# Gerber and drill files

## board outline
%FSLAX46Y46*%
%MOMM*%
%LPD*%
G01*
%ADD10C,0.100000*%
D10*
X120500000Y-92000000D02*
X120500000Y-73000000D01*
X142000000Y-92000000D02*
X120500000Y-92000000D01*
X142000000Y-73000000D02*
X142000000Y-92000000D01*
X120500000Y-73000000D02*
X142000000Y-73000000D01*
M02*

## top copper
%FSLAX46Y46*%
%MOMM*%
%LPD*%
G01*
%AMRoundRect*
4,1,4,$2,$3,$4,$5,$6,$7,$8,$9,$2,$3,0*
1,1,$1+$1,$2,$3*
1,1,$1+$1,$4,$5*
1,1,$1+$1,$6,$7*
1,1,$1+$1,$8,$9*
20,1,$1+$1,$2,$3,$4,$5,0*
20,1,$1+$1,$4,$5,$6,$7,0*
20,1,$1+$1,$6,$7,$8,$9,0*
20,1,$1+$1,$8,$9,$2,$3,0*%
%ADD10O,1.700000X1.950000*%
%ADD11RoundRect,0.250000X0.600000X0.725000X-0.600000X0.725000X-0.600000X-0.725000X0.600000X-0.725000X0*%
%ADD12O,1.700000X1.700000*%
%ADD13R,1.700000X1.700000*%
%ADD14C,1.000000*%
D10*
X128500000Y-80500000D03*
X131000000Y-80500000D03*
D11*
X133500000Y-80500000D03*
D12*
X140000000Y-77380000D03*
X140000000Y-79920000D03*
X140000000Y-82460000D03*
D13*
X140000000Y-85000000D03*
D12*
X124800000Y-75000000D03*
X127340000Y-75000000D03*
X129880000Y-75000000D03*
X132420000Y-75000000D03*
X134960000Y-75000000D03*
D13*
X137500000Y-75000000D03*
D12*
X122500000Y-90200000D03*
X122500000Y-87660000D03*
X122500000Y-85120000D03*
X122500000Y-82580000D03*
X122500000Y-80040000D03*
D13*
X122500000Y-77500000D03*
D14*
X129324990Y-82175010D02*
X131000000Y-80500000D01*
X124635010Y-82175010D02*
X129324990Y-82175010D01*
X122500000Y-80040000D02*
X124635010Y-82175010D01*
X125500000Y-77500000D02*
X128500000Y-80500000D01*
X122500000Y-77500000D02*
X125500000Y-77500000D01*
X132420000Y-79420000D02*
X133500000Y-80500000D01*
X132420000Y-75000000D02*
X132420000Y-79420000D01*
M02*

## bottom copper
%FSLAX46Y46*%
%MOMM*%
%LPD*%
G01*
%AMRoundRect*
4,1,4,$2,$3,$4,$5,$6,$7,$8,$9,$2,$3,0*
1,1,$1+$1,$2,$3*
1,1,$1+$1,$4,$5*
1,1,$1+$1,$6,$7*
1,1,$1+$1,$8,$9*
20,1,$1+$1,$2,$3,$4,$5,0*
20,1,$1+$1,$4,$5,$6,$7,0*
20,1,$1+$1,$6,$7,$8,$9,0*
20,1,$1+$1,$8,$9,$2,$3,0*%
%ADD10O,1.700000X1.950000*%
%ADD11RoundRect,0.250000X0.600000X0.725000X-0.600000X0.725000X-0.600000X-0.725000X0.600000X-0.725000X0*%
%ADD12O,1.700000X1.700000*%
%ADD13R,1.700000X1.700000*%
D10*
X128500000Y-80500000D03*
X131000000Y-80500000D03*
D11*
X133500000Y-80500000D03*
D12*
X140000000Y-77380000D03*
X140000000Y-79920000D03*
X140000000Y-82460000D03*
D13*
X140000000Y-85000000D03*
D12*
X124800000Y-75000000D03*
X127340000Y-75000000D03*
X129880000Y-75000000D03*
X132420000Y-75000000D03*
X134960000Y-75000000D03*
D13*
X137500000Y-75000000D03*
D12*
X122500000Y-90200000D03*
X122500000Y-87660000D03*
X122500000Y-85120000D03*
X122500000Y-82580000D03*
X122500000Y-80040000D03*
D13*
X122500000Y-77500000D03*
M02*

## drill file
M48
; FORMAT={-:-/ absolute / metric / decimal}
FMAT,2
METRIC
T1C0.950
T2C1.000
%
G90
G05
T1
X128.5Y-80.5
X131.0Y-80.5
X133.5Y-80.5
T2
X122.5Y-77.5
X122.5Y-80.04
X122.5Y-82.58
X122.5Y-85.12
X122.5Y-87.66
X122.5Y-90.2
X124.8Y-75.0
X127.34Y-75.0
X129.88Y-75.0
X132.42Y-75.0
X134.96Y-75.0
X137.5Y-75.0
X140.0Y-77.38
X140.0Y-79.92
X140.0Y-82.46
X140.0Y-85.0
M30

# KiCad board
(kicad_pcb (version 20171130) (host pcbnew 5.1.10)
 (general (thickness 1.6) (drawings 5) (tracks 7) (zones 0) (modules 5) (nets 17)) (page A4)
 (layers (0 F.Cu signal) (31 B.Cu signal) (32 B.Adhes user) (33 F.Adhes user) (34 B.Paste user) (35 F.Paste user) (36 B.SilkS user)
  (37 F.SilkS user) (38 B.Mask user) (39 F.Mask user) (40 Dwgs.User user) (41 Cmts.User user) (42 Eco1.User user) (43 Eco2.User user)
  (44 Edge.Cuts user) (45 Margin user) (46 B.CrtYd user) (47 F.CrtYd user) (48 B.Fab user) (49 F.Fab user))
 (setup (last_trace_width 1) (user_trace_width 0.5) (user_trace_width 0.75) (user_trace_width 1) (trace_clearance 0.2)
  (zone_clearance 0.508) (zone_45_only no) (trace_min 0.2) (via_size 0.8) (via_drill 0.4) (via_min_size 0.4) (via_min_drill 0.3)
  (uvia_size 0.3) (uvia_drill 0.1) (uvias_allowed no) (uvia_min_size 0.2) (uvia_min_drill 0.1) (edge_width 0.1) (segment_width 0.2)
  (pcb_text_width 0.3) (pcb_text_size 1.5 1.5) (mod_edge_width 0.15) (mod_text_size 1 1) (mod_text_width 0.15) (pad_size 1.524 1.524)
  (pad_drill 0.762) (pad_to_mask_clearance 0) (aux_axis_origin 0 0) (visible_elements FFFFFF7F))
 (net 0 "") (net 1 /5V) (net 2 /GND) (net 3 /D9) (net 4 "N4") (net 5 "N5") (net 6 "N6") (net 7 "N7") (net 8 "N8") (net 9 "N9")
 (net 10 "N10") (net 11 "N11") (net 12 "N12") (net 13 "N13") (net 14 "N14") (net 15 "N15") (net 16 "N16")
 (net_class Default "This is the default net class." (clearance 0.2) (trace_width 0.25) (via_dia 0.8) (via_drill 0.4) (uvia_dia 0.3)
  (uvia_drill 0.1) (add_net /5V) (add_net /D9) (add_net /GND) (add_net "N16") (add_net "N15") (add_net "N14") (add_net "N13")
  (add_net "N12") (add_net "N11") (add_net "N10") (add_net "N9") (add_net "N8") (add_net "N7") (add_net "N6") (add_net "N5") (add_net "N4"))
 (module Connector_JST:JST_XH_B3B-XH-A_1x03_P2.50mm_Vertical (layer F.Cu) (at 133.5 80.5 180)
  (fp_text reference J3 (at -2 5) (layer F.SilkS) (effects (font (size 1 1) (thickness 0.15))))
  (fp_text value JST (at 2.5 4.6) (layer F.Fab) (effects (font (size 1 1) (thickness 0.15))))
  (pad 3 thru_hole oval (at 5 0 180) (size 1.7 1.95) (drill 0.95) (layers *.Cu *.Mask) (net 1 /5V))
  (pad 2 thru_hole oval (at 2.5 0 180) (size 1.7 1.95) (drill 0.95) (layers *.Cu *.Mask) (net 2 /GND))
  (pad 1 thru_hole roundrect (at 0 0 180) (size 1.7 1.95) (drill 0.95) (layers *.Cu *.Mask) (roundrect_rratio 0.147059) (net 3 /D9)))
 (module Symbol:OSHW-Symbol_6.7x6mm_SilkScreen (layer F.Cu) (at 129 86.5)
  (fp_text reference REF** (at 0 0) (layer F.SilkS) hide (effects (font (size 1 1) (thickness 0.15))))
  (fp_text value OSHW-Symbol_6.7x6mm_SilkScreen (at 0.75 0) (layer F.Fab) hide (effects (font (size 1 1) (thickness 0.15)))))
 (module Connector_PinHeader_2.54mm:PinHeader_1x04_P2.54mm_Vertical (layer B.Cu) (at 140 85)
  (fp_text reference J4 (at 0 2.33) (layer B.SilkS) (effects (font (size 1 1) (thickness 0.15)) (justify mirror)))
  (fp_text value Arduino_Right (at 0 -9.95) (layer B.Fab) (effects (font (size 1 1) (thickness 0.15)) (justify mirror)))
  (pad 4 thru_hole oval (at 0 -7.62) (size 1.7 1.7) (drill 1) (layers *.Cu *.Mask) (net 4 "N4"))
  (pad 3 thru_hole oval (at 0 -5.08) (size 1.7 1.7) (drill 1) (layers *.Cu *.Mask) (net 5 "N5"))
  (pad 2 thru_hole oval (at 0 -2.54) (size 1.7 1.7) (drill 1) (layers *.Cu *.Mask) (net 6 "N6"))
  (pad 1 thru_hole rect (at 0 0) (size 1.7 1.7) (drill 1) (layers *.Cu *.Mask) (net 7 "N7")))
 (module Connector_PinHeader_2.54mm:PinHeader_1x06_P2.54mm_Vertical (layer B.Cu) (at 137.5 75 90)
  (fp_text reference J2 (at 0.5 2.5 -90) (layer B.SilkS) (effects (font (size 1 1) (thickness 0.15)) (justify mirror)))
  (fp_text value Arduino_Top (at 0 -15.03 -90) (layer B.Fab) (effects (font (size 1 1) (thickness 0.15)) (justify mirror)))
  (pad 6 thru_hole oval (at 0 -12.7 90) (size 1.7 1.7) (drill 1) (layers *.Cu *.Mask) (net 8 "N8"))
  (pad 5 thru_hole oval (at 0 -10.16 90) (size 1.7 1.7) (drill 1) (layers *.Cu *.Mask) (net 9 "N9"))
  (pad 4 thru_hole oval (at 0 -7.62 90) (size 1.7 1.7) (drill 1) (layers *.Cu *.Mask) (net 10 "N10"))
  (pad 3 thru_hole oval (at 0 -5.08 90) (size 1.7 1.7) (drill 1) (layers *.Cu *.Mask) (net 3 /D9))
  (pad 2 thru_hole oval (at 0 -2.54 90) (size 1.7 1.7) (drill 1) (layers *.Cu *.Mask) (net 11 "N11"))
  (pad 1 thru_hole rect (at 0 0 90) (size 1.7 1.7) (drill 1) (layers *.Cu *.Mask) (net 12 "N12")))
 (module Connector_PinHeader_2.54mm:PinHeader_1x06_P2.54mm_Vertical (layer B.Cu) (at 122.5 77.5 180)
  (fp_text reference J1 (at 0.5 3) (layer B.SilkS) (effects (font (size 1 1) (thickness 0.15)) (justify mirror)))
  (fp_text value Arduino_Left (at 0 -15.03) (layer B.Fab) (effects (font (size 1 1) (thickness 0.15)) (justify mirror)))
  (pad 6 thru_hole oval (at 0 -12.7 180) (size 1.7 1.7) (drill 1) (layers *.Cu *.Mask) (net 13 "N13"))
  (pad 5 thru_hole oval (at 0 -10.16 180) (size 1.7 1.7) (drill 1) (layers *.Cu *.Mask) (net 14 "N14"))
  (pad 4 thru_hole oval (at 0 -7.62 180) (size 1.7 1.7) (drill 1) (layers *.Cu *.Mask) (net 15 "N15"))
  (pad 3 thru_hole oval (at 0 -5.08 180) (size 1.7 1.7) (drill 1) (layers *.Cu *.Mask) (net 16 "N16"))
  (pad 2 thru_hole oval (at 0 -2.54 180) (size 1.7 1.7) (drill 1) (layers *.Cu *.Mask) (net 2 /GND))
  (pad 1 thru_hole rect (at 0 0 180) (size 1.7 1.7) (drill 1) (layers *.Cu *.Mask) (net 1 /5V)))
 (gr_line (start 120.5 92) (end 120.5 73) (layer Edge.Cuts) (width 0.1))
 (gr_line (start 142 92) (end 120.5 92) (layer Edge.Cuts) (width 0.1))
 (gr_line (start 142 73) (end 142 92) (layer Edge.Cuts) (width 0.1))
 (gr_line (start 120.5 73) (end 142 73) (layer Edge.Cuts) (width 0.1))
 (segment (start 129.32499 82.17501) (end 131 80.5) (width 1) (layer F.Cu) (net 2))
 (segment (start 124.63501 82.17501) (end 129.32499 82.17501) (width 1) (layer F.Cu) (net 2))
 (segment (start 122.5 80.04) (end 124.63501 82.17501) (width 1) (layer F.Cu) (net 2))
 (segment (start 125.5 77.5) (end 128.5 80.5) (width 1) (layer F.Cu) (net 1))
 (segment (start 122.5 77.5) (end 125.5 77.5) (width 1) (layer F.Cu) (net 1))
 (segment (start 132.42 79.42) (end 133.5 80.5) (width 1) (layer F.Cu) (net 3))
 (segment (start 132.42 75) (end 132.42 79.42) (width 1) (layer F.Cu) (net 3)))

